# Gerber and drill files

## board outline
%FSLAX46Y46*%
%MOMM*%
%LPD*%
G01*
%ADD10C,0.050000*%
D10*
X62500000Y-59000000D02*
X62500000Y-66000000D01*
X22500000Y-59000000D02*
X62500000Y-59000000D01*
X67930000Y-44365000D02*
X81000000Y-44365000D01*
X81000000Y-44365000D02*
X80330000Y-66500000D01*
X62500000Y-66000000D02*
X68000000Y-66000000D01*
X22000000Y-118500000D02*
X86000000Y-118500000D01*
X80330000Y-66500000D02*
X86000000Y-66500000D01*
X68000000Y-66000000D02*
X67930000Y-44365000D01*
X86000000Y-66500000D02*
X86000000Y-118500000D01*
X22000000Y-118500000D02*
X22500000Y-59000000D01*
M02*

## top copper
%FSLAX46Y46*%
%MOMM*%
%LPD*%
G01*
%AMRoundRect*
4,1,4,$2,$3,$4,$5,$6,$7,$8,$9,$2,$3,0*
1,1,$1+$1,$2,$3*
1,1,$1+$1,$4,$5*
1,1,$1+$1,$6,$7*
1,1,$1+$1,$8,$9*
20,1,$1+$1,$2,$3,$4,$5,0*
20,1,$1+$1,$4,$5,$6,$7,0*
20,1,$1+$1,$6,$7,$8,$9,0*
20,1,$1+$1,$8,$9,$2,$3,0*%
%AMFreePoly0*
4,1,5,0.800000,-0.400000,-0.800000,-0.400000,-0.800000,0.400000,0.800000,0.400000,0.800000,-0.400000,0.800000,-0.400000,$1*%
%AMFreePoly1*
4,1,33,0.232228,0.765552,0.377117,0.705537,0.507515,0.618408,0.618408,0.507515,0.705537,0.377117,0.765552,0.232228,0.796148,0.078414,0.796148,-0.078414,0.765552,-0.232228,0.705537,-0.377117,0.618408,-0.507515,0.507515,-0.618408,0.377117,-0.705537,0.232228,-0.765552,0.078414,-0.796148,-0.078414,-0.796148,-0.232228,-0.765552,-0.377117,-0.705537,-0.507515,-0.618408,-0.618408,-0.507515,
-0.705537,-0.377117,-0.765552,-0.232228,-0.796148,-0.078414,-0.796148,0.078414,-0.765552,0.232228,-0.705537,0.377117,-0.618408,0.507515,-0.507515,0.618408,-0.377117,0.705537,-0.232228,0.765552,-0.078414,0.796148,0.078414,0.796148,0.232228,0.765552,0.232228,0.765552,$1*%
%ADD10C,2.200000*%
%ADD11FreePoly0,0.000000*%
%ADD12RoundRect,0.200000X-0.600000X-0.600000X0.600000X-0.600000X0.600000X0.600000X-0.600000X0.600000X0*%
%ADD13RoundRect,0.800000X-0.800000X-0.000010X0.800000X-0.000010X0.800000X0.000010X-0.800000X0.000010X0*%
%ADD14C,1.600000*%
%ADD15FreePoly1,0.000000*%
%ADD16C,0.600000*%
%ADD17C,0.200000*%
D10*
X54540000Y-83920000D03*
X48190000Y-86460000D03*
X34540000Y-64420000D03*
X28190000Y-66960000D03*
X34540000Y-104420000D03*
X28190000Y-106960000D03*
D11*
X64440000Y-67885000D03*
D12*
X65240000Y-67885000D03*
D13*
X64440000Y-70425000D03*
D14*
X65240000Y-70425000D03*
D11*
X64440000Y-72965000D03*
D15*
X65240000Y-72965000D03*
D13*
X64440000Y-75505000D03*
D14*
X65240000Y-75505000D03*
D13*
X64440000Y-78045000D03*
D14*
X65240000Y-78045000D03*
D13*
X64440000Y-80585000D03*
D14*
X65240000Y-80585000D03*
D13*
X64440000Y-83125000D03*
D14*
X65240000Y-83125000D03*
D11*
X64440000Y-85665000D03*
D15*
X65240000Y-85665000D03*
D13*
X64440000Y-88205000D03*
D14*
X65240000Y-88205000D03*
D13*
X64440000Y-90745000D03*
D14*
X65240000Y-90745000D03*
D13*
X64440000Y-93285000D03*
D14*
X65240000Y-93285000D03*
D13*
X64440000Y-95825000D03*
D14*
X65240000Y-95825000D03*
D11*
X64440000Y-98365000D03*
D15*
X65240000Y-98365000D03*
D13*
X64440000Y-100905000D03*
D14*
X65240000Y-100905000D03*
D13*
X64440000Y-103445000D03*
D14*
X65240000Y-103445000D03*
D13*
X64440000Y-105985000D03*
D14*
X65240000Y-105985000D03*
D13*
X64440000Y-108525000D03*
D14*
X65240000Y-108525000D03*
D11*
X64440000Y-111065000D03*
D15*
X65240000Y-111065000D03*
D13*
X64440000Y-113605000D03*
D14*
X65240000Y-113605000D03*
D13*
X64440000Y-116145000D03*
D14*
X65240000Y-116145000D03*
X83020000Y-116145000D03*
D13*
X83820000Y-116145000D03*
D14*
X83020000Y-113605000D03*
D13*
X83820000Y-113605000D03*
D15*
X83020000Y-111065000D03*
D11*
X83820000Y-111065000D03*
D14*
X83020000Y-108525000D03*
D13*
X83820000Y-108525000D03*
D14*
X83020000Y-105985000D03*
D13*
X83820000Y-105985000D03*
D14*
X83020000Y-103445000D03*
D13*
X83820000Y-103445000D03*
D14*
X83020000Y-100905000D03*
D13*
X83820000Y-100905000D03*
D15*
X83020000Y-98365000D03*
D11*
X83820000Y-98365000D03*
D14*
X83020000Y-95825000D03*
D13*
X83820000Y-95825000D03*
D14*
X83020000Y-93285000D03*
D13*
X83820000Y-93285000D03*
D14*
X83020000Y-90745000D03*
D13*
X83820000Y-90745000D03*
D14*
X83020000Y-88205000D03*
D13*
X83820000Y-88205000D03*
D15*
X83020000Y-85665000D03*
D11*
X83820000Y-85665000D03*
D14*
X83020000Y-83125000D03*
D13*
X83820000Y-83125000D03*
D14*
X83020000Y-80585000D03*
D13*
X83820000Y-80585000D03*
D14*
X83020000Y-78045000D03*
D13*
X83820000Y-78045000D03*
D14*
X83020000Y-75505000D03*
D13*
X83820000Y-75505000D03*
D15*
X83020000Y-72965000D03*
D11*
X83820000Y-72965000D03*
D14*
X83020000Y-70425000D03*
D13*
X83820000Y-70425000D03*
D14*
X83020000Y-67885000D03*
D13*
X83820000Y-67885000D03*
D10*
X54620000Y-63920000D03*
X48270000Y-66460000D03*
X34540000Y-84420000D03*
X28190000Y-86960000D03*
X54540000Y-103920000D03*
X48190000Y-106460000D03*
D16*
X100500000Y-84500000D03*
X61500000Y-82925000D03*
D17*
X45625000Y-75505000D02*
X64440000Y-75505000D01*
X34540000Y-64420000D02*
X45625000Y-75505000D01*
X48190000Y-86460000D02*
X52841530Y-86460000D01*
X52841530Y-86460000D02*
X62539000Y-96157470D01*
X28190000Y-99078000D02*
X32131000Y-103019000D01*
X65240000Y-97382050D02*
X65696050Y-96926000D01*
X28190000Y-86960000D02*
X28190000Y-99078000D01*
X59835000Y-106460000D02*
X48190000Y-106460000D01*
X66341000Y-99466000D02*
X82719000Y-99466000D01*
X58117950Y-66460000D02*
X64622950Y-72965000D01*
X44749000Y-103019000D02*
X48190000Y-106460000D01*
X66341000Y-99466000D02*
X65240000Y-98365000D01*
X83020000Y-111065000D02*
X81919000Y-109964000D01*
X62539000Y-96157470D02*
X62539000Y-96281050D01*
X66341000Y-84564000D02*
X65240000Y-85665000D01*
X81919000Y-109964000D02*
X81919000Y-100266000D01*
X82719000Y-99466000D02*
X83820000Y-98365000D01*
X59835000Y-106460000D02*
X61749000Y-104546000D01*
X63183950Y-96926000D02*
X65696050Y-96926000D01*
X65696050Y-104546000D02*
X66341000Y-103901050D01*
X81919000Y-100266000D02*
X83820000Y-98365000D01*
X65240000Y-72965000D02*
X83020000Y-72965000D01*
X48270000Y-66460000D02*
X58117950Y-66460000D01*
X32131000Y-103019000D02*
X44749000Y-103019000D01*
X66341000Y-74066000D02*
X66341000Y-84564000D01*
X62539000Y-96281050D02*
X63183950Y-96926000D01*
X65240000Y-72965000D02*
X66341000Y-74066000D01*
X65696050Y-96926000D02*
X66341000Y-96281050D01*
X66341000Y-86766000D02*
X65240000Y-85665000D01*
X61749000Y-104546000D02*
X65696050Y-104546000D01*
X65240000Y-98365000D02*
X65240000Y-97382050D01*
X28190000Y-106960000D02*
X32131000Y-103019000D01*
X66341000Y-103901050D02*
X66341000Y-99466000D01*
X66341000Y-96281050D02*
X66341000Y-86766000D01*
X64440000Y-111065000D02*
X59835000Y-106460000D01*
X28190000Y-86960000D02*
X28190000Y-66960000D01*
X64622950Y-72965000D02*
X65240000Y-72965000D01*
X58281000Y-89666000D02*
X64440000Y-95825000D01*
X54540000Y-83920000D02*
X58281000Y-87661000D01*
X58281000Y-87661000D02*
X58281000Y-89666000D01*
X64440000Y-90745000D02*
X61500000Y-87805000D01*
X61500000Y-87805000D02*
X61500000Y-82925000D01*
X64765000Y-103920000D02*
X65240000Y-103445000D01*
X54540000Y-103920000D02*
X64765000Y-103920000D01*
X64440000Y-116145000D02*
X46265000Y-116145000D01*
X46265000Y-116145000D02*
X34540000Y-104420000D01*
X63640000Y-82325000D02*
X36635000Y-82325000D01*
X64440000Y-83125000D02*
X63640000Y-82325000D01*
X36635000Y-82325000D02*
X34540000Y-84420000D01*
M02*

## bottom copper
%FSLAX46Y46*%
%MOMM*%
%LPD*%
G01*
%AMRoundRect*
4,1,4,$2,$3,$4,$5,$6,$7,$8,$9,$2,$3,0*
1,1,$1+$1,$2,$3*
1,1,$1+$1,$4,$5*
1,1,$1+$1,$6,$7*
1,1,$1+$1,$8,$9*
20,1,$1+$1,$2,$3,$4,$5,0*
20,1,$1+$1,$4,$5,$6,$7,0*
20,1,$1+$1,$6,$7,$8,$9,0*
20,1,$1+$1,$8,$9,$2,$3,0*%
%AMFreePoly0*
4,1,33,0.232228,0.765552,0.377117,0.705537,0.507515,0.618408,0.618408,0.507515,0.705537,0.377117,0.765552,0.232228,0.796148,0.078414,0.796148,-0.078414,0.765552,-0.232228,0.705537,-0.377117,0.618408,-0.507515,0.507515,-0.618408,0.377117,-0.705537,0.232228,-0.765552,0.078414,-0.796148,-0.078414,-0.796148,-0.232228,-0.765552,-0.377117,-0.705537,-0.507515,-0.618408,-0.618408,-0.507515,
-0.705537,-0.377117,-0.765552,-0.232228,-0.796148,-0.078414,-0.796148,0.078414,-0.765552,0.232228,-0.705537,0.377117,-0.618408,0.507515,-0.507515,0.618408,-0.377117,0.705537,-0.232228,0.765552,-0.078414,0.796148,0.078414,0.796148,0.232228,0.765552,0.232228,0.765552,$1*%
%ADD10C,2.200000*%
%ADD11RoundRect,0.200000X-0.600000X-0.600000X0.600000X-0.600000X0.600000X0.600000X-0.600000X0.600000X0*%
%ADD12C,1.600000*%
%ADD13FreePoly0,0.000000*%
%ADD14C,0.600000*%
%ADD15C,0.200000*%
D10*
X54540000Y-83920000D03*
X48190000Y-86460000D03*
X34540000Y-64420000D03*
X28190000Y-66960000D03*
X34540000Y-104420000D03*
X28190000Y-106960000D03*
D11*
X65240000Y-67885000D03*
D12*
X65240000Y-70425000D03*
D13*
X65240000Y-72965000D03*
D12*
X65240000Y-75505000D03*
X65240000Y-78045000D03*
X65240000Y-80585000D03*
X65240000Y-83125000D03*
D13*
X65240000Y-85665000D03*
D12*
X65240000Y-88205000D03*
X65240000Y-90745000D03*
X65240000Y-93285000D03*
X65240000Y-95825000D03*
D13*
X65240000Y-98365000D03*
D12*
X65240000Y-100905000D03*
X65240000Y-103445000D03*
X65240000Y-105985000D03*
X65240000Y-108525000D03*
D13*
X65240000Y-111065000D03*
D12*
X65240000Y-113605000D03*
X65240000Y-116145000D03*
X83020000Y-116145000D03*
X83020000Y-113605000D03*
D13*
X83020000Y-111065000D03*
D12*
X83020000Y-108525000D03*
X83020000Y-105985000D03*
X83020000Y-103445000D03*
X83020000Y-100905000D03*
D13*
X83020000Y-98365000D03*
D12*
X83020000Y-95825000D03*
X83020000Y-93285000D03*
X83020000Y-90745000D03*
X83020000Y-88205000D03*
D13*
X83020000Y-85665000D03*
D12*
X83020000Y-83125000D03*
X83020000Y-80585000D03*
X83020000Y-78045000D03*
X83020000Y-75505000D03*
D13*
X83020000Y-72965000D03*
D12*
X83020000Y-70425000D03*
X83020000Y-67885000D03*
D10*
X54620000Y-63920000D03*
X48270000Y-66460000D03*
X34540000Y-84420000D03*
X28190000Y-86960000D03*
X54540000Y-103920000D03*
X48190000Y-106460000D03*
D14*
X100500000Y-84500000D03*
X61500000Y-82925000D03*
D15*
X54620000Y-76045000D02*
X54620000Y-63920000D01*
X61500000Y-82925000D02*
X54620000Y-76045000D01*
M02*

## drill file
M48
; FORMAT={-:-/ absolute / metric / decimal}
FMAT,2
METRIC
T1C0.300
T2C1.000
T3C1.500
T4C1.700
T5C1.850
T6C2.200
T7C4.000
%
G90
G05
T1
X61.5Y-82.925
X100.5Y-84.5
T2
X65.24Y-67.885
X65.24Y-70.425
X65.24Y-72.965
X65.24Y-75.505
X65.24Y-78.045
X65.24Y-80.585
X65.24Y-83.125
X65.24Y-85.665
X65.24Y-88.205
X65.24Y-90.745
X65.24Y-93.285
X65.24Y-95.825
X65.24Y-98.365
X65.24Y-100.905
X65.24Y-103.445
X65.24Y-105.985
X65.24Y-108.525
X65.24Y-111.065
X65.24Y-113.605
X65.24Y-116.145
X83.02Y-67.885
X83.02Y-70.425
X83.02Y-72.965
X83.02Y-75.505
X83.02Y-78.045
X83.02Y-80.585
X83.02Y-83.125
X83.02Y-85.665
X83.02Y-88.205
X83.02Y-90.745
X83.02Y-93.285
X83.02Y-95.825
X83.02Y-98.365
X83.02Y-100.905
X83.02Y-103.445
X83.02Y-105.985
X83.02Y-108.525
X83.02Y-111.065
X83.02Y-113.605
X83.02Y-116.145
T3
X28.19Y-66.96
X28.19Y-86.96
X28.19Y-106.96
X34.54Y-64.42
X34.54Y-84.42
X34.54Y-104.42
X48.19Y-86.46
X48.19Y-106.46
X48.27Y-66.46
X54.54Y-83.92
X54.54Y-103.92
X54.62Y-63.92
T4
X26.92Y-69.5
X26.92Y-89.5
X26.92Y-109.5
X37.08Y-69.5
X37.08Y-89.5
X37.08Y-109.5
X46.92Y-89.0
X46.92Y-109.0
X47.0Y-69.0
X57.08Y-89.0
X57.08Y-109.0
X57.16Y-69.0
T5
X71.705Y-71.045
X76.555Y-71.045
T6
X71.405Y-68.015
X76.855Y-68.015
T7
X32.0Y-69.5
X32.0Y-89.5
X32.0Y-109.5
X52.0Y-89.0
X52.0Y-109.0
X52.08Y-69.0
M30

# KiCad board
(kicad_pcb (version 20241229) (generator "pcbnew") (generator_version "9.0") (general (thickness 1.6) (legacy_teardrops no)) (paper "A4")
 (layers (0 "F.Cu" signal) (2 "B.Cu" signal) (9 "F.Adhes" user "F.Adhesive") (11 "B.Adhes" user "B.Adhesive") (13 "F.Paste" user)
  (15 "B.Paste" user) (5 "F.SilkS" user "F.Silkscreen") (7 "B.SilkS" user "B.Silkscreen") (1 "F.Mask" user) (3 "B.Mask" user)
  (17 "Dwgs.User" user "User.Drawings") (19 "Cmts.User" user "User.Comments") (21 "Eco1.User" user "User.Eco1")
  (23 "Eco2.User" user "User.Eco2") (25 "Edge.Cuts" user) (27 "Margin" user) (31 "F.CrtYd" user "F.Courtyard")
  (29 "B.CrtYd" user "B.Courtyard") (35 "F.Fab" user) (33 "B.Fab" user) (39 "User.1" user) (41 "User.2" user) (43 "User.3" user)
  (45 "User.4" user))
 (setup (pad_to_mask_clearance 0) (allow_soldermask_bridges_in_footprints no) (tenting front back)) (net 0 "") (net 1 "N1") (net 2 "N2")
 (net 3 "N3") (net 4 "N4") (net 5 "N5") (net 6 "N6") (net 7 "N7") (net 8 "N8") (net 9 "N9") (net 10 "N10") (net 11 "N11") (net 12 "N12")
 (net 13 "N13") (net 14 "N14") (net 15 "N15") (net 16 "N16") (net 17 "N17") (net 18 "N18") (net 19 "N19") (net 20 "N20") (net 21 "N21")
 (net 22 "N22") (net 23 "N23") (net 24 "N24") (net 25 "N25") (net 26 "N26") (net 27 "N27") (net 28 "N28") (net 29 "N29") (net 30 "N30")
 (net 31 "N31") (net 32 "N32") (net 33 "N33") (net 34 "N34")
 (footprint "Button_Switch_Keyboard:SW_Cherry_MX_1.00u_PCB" (layer "F.Cu") (at 54.54 83.92)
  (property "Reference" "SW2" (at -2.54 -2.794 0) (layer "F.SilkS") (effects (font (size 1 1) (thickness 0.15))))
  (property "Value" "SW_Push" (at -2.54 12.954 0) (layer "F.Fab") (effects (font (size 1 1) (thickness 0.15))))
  (pad "" np_thru_hole circle (at -7.62 5.08) (size 1.7 1.7) (drill 1.7) (layers "*.Cu" "*.Mask"))
  (pad "" np_thru_hole circle (at -2.54 5.08) (size 4 4) (drill 4) (layers "*.Cu" "*.Mask"))
  (pad "" np_thru_hole circle (at 2.54 5.08) (size 1.7 1.7) (drill 1.7) (layers "*.Cu" "*.Mask"))
  (pad "1" thru_hole circle (at 0 0) (size 2.2 2.2) (drill 1.5) (layers "*.Cu" "*.Mask") (remove_unused_layers no) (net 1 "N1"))
  (pad "2" thru_hole circle (at -6.35 2.54) (size 2.2 2.2) (drill 1.5) (layers "*.Cu" "*.Mask") (remove_unused_layers no) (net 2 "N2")))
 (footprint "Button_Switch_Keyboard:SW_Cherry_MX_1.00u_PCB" (layer "F.Cu") (at 34.54 64.42)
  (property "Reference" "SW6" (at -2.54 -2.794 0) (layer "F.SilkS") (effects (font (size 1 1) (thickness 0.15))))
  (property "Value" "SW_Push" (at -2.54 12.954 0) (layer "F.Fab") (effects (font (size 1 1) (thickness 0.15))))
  (pad "" np_thru_hole circle (at -7.62 5.08) (size 1.7 1.7) (drill 1.7) (layers "*.Cu" "*.Mask"))
  (pad "" np_thru_hole circle (at -2.54 5.08) (size 4 4) (drill 4) (layers "*.Cu" "*.Mask"))
  (pad "" np_thru_hole circle (at 2.54 5.08) (size 1.7 1.7) (drill 1.7) (layers "*.Cu" "*.Mask"))
  (pad "1" thru_hole circle (at 0 0) (size 2.2 2.2) (drill 1.5) (layers "*.Cu" "*.Mask") (remove_unused_layers no) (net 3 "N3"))
  (pad "2" thru_hole circle (at -6.35 2.54) (size 2.2 2.2) (drill 1.5) (layers "*.Cu" "*.Mask") (remove_unused_layers no) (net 2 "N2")))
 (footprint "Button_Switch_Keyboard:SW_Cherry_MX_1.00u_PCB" (layer "F.Cu") (at 34.54 104.42)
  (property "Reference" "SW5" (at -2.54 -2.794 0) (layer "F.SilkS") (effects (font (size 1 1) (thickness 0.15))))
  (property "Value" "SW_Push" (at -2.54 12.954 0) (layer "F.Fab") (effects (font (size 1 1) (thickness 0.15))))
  (pad "" np_thru_hole circle (at -7.62 5.08) (size 1.7 1.7) (drill 1.7) (layers "*.Cu" "*.Mask"))
  (pad "" np_thru_hole circle (at -2.54 5.08) (size 4 4) (drill 4) (layers "*.Cu" "*.Mask"))
  (pad "" np_thru_hole circle (at 2.54 5.08) (size 1.7 1.7) (drill 1.7) (layers "*.Cu" "*.Mask"))
  (pad "1" thru_hole circle (at 0 0) (size 2.2 2.2) (drill 1.5) (layers "*.Cu" "*.Mask") (remove_unused_layers no) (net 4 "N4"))
  (pad "2" thru_hole circle (at -6.35 2.54) (size 2.2 2.2) (drill 1.5) (layers "*.Cu" "*.Mask") (remove_unused_layers no) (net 2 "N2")))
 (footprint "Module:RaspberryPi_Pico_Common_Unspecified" (layer "F.Cu") (at 74.13 92.015)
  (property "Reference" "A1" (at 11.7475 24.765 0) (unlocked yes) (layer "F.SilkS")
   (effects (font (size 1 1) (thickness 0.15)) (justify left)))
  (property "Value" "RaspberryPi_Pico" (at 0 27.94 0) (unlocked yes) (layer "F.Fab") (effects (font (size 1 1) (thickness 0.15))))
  (pad "" np_thru_hole circle (at -2.725 -24) (size 2.2 2.2) (drill 2.2) (layers "*.Mask"))
  (pad "" np_thru_hole circle (at -2.425 -20.97) (size 1.85 1.85) (drill 1.85) (layers "*.Mask"))
  (pad "" np_thru_hole circle (at 2.425 -20.97) (size 1.85 1.85) (drill 1.85) (layers "*.Mask"))
  (pad "" np_thru_hole circle (at 2.725 -24) (size 2.2 2.2) (drill 2.2) (layers "*.Mask"))
  (pad "1" smd custom (at -9.69 -24.13) (size 1.6 0.8) (layers "F.Cu" "F.Mask") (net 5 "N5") (options (clearance outline) (anchor rect))
   (primitives))
  (pad "1" thru_hole roundrect (at -8.89 -24.13) (size 1.6 1.6) (drill 1) (layers "*.Cu" "*.Mask") (remove_unused_layers no)
   (roundrect_rratio 0.125) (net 5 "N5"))
  (pad "2" smd roundrect (at -9.69 -21.59) (size 3.2 1.6) (layers "F.Cu" "F.Mask") (roundrect_rratio 0.5) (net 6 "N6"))
  (pad "2" thru_hole circle (at -8.89 -21.59) (size 1.6 1.6) (drill 1) (layers "*.Cu" "*.Mask") (remove_unused_layers no) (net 6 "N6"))
  (pad "3" smd custom (at -9.69 -19.05) (size 1.6 0.8) (layers "F.Cu" "F.Mask") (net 2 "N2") (options (clearance outline) (anchor rect))
   (primitives))
  (pad "3" thru_hole custom (at -8.89 -19.05) (size 1.6 1.6) (drill 1) (layers "*.Cu" "*.Mask") (remove_unused_layers no) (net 2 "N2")
   (options (clearance outline) (anchor circle)) (primitives))
  (pad "4" smd roundrect (at -9.69 -16.51) (size 3.2 1.6) (layers "F.Cu" "F.Mask") (roundrect_rratio 0.5) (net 3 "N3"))
  (pad "4" thru_hole circle (at -8.89 -16.51) (size 1.6 1.6) (drill 1) (layers "*.Cu" "*.Mask") (remove_unused_layers no) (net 3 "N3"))
  (pad "5" smd roundrect (at -9.69 -13.97) (size 3.2 1.6) (layers "F.Cu" "F.Mask") (roundrect_rratio 0.5) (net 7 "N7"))
  (pad "5" thru_hole circle (at -8.89 -13.97) (size 1.6 1.6) (drill 1) (layers "*.Cu" "*.Mask") (remove_unused_layers no) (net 7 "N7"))
  (pad "6" smd roundrect (at -9.69 -11.43) (size 3.2 1.6) (layers "F.Cu" "F.Mask") (roundrect_rratio 0.5) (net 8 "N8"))
  (pad "6" thru_hole circle (at -8.89 -11.43) (size 1.6 1.6) (drill 1) (layers "*.Cu" "*.Mask") (remove_unused_layers no) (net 8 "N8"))
  (pad "7" smd roundrect (at -9.69 -8.89) (size 3.2 1.6) (layers "F.Cu" "F.Mask") (roundrect_rratio 0.5) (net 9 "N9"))
  (pad "7" thru_hole circle (at -8.89 -8.89) (size 1.6 1.6) (drill 1) (layers "*.Cu" "*.Mask") (remove_unused_layers no) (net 9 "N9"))
  (pad "8" smd custom (at -9.69 -6.35) (size 1.6 0.8) (layers "F.Cu" "F.Mask") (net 2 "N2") (options (clearance outline) (anchor rect))
   (primitives))
  (pad "8" thru_hole custom (at -8.89 -6.35) (size 1.6 1.6) (drill 1) (layers "*.Cu" "*.Mask") (remove_unused_layers no) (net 2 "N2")
   (options (clearance outline) (anchor circle)) (primitives))
  (pad "9" smd roundrect (at -9.69 -3.81) (size 3.2 1.6) (layers "F.Cu" "F.Mask") (roundrect_rratio 0.5) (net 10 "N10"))
  (pad "9" thru_hole circle (at -8.89 -3.81) (size 1.6 1.6) (drill 1) (layers "*.Cu" "*.Mask") (remove_unused_layers no) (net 10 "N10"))
  (pad "10" smd roundrect (at -9.69 -1.27) (size 3.2 1.6) (layers "F.Cu" "F.Mask") (roundrect_rratio 0.5) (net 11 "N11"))
  (pad "10" thru_hole circle (at -8.89 -1.27) (size 1.6 1.6) (drill 1) (layers "*.Cu" "*.Mask") (remove_unused_layers no) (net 11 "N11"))
  (pad "11" smd roundrect (at -9.69 1.27) (size 3.2 1.6) (layers "F.Cu" "F.Mask") (roundrect_rratio 0.5) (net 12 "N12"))
  (pad "11" thru_hole circle (at -8.89 1.27) (size 1.6 1.6) (drill 1) (layers "*.Cu" "*.Mask") (remove_unused_layers no) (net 12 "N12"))
  (pad "12" smd roundrect (at -9.69 3.81) (size 3.2 1.6) (layers "F.Cu" "F.Mask") (roundrect_rratio 0.5) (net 1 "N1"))
  (pad "12" thru_hole circle (at -8.89 3.81) (size 1.6 1.6) (drill 1) (layers "*.Cu" "*.Mask") (remove_unused_layers no) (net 1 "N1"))
  (pad "13" smd custom (at -9.69 6.35) (size 1.6 0.8) (layers "F.Cu" "F.Mask") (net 2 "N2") (options (clearance outline) (anchor rect))
   (primitives))
  (pad "13" thru_hole custom (at -8.89 6.35) (size 1.6 1.6) (drill 1) (layers "*.Cu" "*.Mask") (remove_unused_layers no) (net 2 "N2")
   (options (clearance outline) (anchor circle)) (primitives))
  (pad "14" smd roundrect (at -9.69 8.89) (size 3.2 1.6) (layers "F.Cu" "F.Mask") (roundrect_rratio 0.5) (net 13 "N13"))
  (pad "14" thru_hole circle (at -8.89 8.89) (size 1.6 1.6) (drill 1) (layers "*.Cu" "*.Mask") (remove_unused_layers no) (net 13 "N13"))
  (pad "15" smd roundrect (at -9.69 11.43) (size 3.2 1.6) (layers "F.Cu" "F.Mask") (roundrect_rratio 0.5) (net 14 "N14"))
  (pad "15" thru_hole circle (at -8.89 11.43) (size 1.6 1.6) (drill 1) (layers "*.Cu" "*.Mask") (remove_unused_layers no) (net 14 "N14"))
  (pad "16" smd roundrect (at -9.69 13.97) (size 3.2 1.6) (layers "F.Cu" "F.Mask") (roundrect_rratio 0.5) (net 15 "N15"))
  (pad "16" thru_hole circle (at -8.89 13.97) (size 1.6 1.6) (drill 1) (layers "*.Cu" "*.Mask") (remove_unused_layers no) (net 15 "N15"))
  (pad "17" smd roundrect (at -9.69 16.51) (size 3.2 1.6) (layers "F.Cu" "F.Mask") (roundrect_rratio 0.5) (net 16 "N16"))
  (pad "17" thru_hole circle (at -8.89 16.51) (size 1.6 1.6) (drill 1) (layers "*.Cu" "*.Mask") (remove_unused_layers no) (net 16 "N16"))
  (pad "18" smd custom (at -9.69 19.05) (size 1.6 0.8) (layers "F.Cu" "F.Mask") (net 2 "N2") (options (clearance outline) (anchor rect))
   (primitives))
  (pad "18" thru_hole custom (at -8.89 19.05) (size 1.6 1.6) (drill 1) (layers "*.Cu" "*.Mask") (remove_unused_layers no) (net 2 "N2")
   (options (clearance outline) (anchor circle)) (primitives))
  (pad "19" smd roundrect (at -9.69 21.59) (size 3.2 1.6) (layers "F.Cu" "F.Mask") (roundrect_rratio 0.5) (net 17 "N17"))
  (pad "19" thru_hole circle (at -8.89 21.59) (size 1.6 1.6) (drill 1) (layers "*.Cu" "*.Mask") (remove_unused_layers no) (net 17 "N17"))
  (pad "20" smd roundrect (at -9.69 24.13) (size 3.2 1.6) (layers "F.Cu" "F.Mask") (roundrect_rratio 0.5) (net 4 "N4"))
  (pad "20" thru_hole circle (at -8.89 24.13) (size 1.6 1.6) (drill 1) (layers "*.Cu" "*.Mask") (remove_unused_layers no) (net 4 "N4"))
  (pad "21" thru_hole circle (at 8.89 24.13) (size 1.6 1.6) (drill 1) (layers "*.Cu" "*.Mask") (remove_unused_layers no) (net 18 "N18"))
  (pad "21" smd roundrect (at 9.69 24.13) (size 3.2 1.6) (layers "F.Cu" "F.Mask") (roundrect_rratio 0.5) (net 18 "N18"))
  (pad "22" thru_hole circle (at 8.89 21.59) (size 1.6 1.6) (drill 1) (layers "*.Cu" "*.Mask") (remove_unused_layers no) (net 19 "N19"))
  (pad "22" smd roundrect (at 9.69 21.59) (size 3.2 1.6) (layers "F.Cu" "F.Mask") (roundrect_rratio 0.5) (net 19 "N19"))
  (pad "23" thru_hole custom (at 8.89 19.05) (size 1.6 1.6) (drill 1) (layers "*.Cu" "*.Mask") (remove_unused_layers no) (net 2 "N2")
   (options (clearance outline) (anchor circle)) (primitives))
  (pad "23" smd custom (at 9.69 19.05) (size 1.6 0.8) (layers "F.Cu" "F.Mask") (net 2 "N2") (options (clearance outline) (anchor rect))
   (primitives))
  (pad "24" thru_hole circle (at 8.89 16.51) (size 1.6 1.6) (drill 1) (layers "*.Cu" "*.Mask") (remove_unused_layers no) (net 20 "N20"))
  (pad "24" smd roundrect (at 9.69 16.51) (size 3.2 1.6) (layers "F.Cu" "F.Mask") (roundrect_rratio 0.5) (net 20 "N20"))
  (pad "25" thru_hole circle (at 8.89 13.97) (size 1.6 1.6) (drill 1) (layers "*.Cu" "*.Mask") (remove_unused_layers no) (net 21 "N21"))
  (pad "25" smd roundrect (at 9.69 13.97) (size 3.2 1.6) (layers "F.Cu" "F.Mask") (roundrect_rratio 0.5) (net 21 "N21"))
  (pad "26" thru_hole circle (at 8.89 11.43) (size 1.6 1.6) (drill 1) (layers "*.Cu" "*.Mask") (remove_unused_layers no) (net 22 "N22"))
  (pad "26" smd roundrect (at 9.69 11.43) (size 3.2 1.6) (layers "F.Cu" "F.Mask") (roundrect_rratio 0.5) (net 22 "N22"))
  (pad "27" thru_hole circle (at 8.89 8.89) (size 1.6 1.6) (drill 1) (layers "*.Cu" "*.Mask") (remove_unused_layers no) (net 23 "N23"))
  (pad "27" smd roundrect (at 9.69 8.89) (size 3.2 1.6) (layers "F.Cu" "F.Mask") (roundrect_rratio 0.5) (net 23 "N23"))
  (pad "28" thru_hole custom (at 8.89 6.35) (size 1.6 1.6) (drill 1) (layers "*.Cu" "*.Mask") (remove_unused_layers no) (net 2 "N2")
   (options (clearance outline) (anchor circle)) (primitives))
  (pad "28" smd custom (at 9.69 6.35) (size 1.6 0.8) (layers "F.Cu" "F.Mask") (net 2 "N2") (options (clearance outline) (anchor rect))
   (primitives))
  (pad "29" thru_hole circle (at 8.89 3.81) (size 1.6 1.6) (drill 1) (layers "*.Cu" "*.Mask") (remove_unused_layers no) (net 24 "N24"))
  (pad "29" smd roundrect (at 9.69 3.81) (size 3.2 1.6) (layers "F.Cu" "F.Mask") (roundrect_rratio 0.5) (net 24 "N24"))
  (pad "30" thru_hole circle (at 8.89 1.27) (size 1.6 1.6) (drill 1) (layers "*.Cu" "*.Mask") (remove_unused_layers no) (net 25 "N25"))
  (pad "30" smd roundrect (at 9.69 1.27) (size 3.2 1.6) (layers "F.Cu" "F.Mask") (roundrect_rratio 0.5) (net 25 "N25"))
  (pad "31" thru_hole circle (at 8.89 -1.27) (size 1.6 1.6) (drill 1) (layers "*.Cu" "*.Mask") (remove_unused_layers no) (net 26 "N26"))
  (pad "31" smd roundrect (at 9.69 -1.27) (size 3.2 1.6) (layers "F.Cu" "F.Mask") (roundrect_rratio 0.5) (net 26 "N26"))
  (pad "32" thru_hole circle (at 8.89 -3.81) (size 1.6 1.6) (drill 1) (layers "*.Cu" "*.Mask") (remove_unused_layers no) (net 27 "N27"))
  (pad "32" smd roundrect (at 9.69 -3.81) (size 3.2 1.6) (layers "F.Cu" "F.Mask") (roundrect_rratio 0.5) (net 27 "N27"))
  (pad "33" thru_hole custom (at 8.89 -6.35) (size 1.6 1.6) (drill 1) (layers "*.Cu" "*.Mask") (remove_unused_layers no) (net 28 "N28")
   (options (clearance outline) (anchor circle)) (primitives))
  (pad "33" smd custom (at 9.69 -6.35) (size 1.6 0.8) (layers "F.Cu" "F.Mask") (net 28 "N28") (options (clearance outline) (anchor rect))
   (primitives))
  (pad "34" thru_hole circle (at 8.89 -8.89) (size 1.6 1.6) (drill 1) (layers "*.Cu" "*.Mask") (remove_unused_layers no) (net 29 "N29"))
  (pad "34" smd roundrect (at 9.69 -8.89) (size 3.2 1.6) (layers "F.Cu" "F.Mask") (roundrect_rratio 0.5) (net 29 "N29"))
  (pad "35" thru_hole circle (at 8.89 -11.43) (size 1.6 1.6) (drill 1) (layers "*.Cu" "*.Mask") (remove_unused_layers no) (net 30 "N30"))
  (pad "35" smd roundrect (at 9.69 -11.43) (size 3.2 1.6) (layers "F.Cu" "F.Mask") (roundrect_rratio 0.5) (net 30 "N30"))
  (pad "36" thru_hole circle (at 8.89 -13.97) (size 1.6 1.6) (drill 1) (layers "*.Cu" "*.Mask") (remove_unused_layers no) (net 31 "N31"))
  (pad "36" smd roundrect (at 9.69 -13.97) (size 3.2 1.6) (layers "F.Cu" "F.Mask") (roundrect_rratio 0.5) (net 31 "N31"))
  (pad "37" thru_hole circle (at 8.89 -16.51) (size 1.6 1.6) (drill 1) (layers "*.Cu" "*.Mask") (remove_unused_layers no) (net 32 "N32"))
  (pad "37" smd roundrect (at 9.69 -16.51) (size 3.2 1.6) (layers "F.Cu" "F.Mask") (roundrect_rratio 0.5) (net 32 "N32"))
  (pad "38" thru_hole custom (at 8.89 -19.05) (size 1.6 1.6) (drill 1) (layers "*.Cu" "*.Mask") (remove_unused_layers no) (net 2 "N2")
   (options (clearance outline) (anchor circle)) (primitives))
  (pad "38" smd custom (at 9.69 -19.05) (size 1.6 0.8) (layers "F.Cu" "F.Mask") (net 2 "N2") (options (clearance outline) (anchor rect))
   (primitives))
  (pad "39" thru_hole circle (at 8.89 -21.59) (size 1.6 1.6) (drill 1) (layers "*.Cu" "*.Mask") (remove_unused_layers no) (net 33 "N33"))
  (pad "39" smd roundrect (at 9.69 -21.59) (size 3.2 1.6) (layers "F.Cu" "F.Mask") (roundrect_rratio 0.5) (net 33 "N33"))
  (pad "40" thru_hole circle (at 8.89 -24.13) (size 1.6 1.6) (drill 1) (layers "*.Cu" "*.Mask") (remove_unused_layers no) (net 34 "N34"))
  (pad "40" smd roundrect (at 9.69 -24.13) (size 3.2 1.6) (layers "F.Cu" "F.Mask") (roundrect_rratio 0.5) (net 34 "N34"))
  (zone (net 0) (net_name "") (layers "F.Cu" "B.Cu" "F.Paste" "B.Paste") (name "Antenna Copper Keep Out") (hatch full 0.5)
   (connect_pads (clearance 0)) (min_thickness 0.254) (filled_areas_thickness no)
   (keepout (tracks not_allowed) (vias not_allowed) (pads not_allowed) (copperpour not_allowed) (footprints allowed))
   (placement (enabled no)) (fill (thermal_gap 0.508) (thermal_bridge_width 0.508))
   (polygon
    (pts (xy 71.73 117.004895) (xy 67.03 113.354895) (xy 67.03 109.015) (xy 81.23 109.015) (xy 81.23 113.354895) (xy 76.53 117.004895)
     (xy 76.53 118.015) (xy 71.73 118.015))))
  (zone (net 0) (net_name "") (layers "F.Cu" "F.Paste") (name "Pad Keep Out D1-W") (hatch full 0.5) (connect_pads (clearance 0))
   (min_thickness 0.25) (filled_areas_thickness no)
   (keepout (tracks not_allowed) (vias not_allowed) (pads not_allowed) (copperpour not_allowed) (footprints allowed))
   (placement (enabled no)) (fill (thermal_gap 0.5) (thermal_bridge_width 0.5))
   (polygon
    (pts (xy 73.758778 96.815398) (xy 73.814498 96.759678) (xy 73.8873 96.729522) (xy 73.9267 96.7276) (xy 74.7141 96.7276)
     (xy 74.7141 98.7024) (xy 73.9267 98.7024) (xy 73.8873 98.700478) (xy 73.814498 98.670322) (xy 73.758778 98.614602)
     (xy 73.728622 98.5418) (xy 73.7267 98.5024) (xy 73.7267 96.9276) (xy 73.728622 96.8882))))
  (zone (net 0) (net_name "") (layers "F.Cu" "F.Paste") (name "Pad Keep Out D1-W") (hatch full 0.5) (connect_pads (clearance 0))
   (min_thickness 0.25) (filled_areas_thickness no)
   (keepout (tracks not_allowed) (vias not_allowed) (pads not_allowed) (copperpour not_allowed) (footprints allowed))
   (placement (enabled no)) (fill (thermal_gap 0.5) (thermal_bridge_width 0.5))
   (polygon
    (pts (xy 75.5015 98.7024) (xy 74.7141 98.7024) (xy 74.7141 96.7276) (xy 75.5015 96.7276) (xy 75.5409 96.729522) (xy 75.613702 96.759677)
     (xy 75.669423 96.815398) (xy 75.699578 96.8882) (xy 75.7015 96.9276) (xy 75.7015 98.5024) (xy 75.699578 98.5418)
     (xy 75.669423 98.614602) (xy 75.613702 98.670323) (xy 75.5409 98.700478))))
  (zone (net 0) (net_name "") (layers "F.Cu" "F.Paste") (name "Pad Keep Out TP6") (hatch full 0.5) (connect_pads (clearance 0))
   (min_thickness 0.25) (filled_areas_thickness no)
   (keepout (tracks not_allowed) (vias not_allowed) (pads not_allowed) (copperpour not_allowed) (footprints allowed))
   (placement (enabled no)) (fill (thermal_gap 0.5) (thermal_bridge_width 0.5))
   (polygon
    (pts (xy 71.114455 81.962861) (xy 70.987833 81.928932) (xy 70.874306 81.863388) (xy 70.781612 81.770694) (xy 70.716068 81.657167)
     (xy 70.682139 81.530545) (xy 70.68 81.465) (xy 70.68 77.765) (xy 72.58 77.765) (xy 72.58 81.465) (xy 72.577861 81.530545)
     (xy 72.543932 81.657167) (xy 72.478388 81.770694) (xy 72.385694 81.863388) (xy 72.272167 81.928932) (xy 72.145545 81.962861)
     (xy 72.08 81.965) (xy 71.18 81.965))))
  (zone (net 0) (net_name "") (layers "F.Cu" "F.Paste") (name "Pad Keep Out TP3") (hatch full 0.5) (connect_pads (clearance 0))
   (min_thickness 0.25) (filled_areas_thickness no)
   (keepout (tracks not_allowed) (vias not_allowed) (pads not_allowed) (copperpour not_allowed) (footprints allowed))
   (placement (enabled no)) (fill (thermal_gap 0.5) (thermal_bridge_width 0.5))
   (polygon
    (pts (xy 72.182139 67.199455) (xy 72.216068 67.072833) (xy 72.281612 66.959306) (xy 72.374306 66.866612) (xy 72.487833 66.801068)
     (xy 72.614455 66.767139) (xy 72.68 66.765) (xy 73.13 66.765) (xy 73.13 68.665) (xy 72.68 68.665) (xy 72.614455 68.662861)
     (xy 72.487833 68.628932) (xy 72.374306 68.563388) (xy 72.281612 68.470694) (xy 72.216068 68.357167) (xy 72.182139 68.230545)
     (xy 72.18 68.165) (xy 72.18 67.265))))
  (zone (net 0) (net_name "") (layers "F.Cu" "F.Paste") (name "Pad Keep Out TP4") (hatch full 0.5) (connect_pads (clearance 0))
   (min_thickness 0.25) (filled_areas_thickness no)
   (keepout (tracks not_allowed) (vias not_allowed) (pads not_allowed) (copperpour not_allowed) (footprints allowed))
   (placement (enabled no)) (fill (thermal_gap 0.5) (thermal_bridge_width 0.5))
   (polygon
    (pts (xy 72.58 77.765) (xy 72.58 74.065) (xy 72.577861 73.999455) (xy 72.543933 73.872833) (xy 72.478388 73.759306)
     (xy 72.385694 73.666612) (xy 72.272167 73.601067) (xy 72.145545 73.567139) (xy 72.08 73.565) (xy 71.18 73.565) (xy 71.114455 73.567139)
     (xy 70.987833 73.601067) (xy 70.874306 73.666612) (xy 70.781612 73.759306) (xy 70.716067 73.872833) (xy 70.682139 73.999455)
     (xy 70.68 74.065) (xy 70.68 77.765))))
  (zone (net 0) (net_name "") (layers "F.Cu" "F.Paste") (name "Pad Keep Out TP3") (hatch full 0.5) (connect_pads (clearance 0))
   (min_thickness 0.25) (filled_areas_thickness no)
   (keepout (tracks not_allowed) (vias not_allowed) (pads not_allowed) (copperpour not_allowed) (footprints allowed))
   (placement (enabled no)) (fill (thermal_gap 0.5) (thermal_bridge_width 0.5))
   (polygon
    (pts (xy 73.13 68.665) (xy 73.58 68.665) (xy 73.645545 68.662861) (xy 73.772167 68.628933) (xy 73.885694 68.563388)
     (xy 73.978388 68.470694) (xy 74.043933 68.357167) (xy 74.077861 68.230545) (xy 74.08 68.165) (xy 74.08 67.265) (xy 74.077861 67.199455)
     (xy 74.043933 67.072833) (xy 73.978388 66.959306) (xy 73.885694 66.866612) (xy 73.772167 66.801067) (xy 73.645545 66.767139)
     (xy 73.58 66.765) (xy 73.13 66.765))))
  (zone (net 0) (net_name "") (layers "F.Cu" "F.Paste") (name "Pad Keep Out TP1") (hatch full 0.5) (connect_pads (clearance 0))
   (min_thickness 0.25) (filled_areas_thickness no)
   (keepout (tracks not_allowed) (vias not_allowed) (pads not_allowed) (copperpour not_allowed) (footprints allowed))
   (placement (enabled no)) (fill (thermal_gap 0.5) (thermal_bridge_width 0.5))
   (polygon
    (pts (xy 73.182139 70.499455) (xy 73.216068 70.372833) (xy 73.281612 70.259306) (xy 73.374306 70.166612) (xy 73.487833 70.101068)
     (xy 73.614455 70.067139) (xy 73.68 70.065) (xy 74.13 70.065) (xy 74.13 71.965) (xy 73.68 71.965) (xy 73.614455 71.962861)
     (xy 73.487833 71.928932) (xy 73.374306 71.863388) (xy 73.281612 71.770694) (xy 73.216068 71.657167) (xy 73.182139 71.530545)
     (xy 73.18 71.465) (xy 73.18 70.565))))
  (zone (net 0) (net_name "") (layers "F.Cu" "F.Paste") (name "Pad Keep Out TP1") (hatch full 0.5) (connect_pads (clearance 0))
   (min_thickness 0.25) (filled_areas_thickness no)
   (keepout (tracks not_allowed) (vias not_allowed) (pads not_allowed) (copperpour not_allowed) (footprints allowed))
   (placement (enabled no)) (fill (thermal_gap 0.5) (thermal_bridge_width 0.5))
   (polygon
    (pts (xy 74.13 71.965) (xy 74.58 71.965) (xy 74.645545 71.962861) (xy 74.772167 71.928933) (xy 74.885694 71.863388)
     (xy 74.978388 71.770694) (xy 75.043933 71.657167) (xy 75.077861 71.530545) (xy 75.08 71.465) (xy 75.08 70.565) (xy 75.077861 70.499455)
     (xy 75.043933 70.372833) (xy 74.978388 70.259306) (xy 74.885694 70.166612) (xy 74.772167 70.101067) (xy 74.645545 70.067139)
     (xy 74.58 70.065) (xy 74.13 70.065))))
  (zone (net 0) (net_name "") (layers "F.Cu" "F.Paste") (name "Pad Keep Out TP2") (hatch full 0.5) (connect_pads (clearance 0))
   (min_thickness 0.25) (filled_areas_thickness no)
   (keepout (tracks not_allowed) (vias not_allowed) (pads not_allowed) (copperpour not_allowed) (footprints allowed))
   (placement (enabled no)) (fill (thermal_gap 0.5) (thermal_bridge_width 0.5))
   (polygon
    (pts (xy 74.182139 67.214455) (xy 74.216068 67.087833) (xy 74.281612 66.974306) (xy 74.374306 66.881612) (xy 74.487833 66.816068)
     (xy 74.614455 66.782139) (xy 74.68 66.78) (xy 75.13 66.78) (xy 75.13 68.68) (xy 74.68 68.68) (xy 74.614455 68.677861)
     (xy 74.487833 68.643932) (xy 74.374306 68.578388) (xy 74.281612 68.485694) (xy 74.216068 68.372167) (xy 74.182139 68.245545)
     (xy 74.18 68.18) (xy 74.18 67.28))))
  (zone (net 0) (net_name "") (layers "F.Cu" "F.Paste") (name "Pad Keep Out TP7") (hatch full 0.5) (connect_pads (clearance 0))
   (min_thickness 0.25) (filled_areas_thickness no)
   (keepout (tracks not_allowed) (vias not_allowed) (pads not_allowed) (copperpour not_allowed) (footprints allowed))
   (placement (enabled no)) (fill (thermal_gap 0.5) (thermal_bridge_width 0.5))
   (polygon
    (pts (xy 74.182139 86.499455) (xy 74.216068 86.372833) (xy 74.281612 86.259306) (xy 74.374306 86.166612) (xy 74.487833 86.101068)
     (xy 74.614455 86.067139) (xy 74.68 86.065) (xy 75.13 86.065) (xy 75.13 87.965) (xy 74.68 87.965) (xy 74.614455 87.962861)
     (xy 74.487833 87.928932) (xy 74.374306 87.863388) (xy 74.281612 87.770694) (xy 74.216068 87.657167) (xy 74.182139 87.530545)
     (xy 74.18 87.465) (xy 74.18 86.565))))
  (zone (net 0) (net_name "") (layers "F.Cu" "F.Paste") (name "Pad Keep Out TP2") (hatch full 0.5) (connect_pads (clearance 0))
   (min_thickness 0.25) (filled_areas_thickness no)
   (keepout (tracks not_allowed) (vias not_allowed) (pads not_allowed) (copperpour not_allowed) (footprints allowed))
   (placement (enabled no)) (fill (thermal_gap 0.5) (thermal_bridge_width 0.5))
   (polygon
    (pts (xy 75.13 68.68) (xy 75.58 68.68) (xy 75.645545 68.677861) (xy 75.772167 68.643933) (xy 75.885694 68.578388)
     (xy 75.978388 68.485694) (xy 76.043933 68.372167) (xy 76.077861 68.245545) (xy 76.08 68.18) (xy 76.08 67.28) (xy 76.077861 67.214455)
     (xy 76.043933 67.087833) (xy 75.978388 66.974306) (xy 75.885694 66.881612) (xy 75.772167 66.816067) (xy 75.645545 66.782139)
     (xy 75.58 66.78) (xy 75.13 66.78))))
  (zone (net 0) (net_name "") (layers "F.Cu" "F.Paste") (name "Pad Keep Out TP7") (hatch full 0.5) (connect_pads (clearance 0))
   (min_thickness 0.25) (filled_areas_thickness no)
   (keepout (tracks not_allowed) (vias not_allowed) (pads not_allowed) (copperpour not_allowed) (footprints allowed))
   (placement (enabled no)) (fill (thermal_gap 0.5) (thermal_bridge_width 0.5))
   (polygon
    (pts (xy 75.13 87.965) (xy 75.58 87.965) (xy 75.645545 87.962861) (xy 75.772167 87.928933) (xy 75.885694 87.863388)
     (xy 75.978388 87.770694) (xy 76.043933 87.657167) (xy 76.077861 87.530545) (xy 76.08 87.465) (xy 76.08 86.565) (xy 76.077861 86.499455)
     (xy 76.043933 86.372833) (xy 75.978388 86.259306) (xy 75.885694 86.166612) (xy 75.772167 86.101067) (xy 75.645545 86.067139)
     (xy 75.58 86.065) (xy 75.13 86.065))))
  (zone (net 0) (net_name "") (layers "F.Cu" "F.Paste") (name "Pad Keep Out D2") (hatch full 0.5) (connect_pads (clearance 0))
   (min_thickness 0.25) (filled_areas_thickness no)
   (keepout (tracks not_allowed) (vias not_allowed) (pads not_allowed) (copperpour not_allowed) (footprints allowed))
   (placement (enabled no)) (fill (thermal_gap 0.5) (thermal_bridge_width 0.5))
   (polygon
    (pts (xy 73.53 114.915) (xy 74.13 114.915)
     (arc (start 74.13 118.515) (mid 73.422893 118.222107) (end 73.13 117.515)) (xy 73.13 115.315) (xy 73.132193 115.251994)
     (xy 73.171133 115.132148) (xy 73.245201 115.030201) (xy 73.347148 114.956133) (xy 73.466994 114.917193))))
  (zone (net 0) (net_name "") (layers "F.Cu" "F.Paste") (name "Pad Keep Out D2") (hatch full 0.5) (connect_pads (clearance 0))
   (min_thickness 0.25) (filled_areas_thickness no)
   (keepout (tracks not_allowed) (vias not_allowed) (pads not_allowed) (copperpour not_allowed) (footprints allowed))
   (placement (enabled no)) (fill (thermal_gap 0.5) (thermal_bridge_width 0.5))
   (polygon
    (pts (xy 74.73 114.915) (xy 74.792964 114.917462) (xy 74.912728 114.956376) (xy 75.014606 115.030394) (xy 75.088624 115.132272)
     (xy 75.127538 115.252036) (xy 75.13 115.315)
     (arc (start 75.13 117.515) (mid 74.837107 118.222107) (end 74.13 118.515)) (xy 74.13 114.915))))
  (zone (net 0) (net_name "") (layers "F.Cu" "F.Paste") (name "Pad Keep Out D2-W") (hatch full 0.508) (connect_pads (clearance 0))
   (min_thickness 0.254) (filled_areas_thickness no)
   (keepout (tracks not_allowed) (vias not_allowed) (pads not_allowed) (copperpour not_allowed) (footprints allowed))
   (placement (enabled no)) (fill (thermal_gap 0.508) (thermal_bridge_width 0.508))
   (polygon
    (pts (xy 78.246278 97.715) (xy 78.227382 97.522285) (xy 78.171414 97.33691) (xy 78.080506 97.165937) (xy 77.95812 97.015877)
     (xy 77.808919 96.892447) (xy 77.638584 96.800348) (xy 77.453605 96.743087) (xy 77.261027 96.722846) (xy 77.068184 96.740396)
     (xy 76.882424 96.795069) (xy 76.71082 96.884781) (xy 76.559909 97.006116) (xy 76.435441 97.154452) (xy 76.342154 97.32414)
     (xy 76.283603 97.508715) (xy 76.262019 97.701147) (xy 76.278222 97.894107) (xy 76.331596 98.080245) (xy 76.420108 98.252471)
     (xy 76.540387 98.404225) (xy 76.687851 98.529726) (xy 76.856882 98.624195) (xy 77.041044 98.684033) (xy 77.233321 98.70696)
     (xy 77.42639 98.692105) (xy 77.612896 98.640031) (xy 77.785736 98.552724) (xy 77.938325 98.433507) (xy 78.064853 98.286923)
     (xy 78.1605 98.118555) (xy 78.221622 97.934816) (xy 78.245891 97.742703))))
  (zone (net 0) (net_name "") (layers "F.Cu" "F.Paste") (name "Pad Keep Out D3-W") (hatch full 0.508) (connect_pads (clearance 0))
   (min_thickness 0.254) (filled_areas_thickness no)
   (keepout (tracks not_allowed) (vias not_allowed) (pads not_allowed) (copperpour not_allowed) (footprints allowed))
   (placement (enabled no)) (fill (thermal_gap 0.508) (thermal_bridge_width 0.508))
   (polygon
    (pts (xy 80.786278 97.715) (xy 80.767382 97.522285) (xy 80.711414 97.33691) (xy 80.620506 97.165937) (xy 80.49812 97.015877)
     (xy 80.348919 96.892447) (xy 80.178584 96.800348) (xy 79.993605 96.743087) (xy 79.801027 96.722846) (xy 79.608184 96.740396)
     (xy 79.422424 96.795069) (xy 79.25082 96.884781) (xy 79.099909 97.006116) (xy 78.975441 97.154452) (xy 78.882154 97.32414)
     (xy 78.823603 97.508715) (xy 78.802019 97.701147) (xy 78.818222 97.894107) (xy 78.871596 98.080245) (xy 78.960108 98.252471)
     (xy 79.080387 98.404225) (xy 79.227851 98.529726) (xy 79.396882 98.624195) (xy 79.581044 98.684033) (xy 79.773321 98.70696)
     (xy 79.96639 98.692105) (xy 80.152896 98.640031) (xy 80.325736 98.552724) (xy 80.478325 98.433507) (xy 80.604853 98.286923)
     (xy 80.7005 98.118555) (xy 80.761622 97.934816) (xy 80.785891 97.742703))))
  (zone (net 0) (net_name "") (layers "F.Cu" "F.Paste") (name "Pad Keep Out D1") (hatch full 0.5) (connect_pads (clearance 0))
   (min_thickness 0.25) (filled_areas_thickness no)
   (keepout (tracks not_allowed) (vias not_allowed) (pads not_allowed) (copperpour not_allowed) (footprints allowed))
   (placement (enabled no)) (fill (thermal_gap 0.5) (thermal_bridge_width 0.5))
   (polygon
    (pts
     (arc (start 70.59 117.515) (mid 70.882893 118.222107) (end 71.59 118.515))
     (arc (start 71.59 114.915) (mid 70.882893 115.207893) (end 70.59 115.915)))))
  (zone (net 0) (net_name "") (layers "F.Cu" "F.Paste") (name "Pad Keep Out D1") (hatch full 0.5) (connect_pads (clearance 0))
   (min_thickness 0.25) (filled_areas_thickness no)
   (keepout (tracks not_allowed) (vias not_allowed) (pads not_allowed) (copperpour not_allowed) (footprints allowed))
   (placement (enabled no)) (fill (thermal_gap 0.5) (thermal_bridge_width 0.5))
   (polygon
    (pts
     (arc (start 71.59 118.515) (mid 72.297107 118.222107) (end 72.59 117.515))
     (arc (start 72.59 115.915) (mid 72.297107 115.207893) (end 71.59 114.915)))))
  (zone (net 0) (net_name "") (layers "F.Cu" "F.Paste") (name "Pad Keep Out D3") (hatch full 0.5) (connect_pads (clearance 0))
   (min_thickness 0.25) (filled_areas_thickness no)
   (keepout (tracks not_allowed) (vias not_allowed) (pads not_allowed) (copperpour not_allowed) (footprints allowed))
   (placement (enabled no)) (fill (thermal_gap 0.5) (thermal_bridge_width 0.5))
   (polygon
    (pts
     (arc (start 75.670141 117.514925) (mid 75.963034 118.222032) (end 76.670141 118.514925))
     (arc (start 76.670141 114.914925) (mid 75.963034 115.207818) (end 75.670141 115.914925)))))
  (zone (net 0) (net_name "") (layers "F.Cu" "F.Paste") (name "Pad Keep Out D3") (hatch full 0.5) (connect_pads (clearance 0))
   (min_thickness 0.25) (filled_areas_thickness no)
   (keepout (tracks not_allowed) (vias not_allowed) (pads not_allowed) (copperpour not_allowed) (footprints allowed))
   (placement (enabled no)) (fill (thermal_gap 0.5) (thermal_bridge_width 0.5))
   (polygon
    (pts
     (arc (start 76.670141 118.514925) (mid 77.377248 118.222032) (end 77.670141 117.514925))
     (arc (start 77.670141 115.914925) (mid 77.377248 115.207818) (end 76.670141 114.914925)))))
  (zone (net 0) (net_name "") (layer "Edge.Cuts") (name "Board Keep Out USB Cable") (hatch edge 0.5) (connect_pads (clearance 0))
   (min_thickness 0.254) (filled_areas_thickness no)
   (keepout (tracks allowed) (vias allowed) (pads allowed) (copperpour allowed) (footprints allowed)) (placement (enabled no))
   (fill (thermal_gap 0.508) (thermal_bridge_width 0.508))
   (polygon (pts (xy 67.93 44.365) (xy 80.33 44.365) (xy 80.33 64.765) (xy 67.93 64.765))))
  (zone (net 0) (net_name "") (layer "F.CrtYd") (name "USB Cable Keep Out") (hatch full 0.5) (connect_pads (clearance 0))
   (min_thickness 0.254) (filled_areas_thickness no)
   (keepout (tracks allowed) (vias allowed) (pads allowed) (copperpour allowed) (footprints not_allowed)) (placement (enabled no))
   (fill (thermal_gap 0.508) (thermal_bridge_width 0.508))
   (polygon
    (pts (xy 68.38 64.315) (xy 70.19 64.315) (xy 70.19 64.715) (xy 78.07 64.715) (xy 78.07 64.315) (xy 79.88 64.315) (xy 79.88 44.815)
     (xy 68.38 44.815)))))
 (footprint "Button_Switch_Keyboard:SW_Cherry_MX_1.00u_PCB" (layer "F.Cu") (at 54.62 63.92)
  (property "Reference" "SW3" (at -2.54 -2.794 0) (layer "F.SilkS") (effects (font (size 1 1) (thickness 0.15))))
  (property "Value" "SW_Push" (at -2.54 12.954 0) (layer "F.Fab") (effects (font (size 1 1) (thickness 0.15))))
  (pad "" np_thru_hole circle (at -7.62 5.08) (size 1.7 1.7) (drill 1.7) (layers "*.Cu" "*.Mask"))
  (pad "" np_thru_hole circle (at -2.54 5.08) (size 4 4) (drill 4) (layers "*.Cu" "*.Mask"))
  (pad "" np_thru_hole circle (at 2.54 5.08) (size 1.7 1.7) (drill 1.7) (layers "*.Cu" "*.Mask"))
  (pad "1" thru_hole circle (at 0 0) (size 2.2 2.2) (drill 1.5) (layers "*.Cu" "*.Mask") (remove_unused_layers no) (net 11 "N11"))
  (pad "2" thru_hole circle (at -6.35 2.54) (size 2.2 2.2) (drill 1.5) (layers "*.Cu" "*.Mask") (remove_unused_layers no) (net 2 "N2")))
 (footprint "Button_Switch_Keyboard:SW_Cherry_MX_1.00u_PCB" (layer "F.Cu") (at 34.54 84.42)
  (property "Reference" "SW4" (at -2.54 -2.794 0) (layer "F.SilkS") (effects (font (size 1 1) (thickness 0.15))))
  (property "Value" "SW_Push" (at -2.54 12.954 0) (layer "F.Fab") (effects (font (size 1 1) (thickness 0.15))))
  (pad "" np_thru_hole circle (at -7.62 5.08) (size 1.7 1.7) (drill 1.7) (layers "*.Cu" "*.Mask"))
  (pad "" np_thru_hole circle (at -2.54 5.08) (size 4 4) (drill 4) (layers "*.Cu" "*.Mask"))
  (pad "" np_thru_hole circle (at 2.54 5.08) (size 1.7 1.7) (drill 1.7) (layers "*.Cu" "*.Mask"))
  (pad "1" thru_hole circle (at 0 0) (size 2.2 2.2) (drill 1.5) (layers "*.Cu" "*.Mask") (remove_unused_layers no) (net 9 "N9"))
  (pad "2" thru_hole circle (at -6.35 2.54) (size 2.2 2.2) (drill 1.5) (layers "*.Cu" "*.Mask") (remove_unused_layers no) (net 2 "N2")))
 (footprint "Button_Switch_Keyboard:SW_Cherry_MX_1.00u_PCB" (layer "F.Cu") (at 54.54 103.92)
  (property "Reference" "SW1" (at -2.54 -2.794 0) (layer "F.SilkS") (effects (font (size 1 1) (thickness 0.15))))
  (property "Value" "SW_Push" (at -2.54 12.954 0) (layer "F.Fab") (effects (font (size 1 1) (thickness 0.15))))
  (pad "" np_thru_hole circle (at -7.62 5.08) (size 1.7 1.7) (drill 1.7) (layers "*.Cu" "*.Mask"))
  (pad "" np_thru_hole circle (at -2.54 5.08) (size 4 4) (drill 4) (layers "*.Cu" "*.Mask"))
  (pad "" np_thru_hole circle (at 2.54 5.08) (size 1.7 1.7) (drill 1.7) (layers "*.Cu" "*.Mask"))
  (pad "1" thru_hole circle (at 0 0) (size 2.2 2.2) (drill 1.5) (layers "*.Cu" "*.Mask") (remove_unused_layers no) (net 14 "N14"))
  (pad "2" thru_hole circle (at -6.35 2.54) (size 2.2 2.2) (drill 1.5) (layers "*.Cu" "*.Mask") (remove_unused_layers no) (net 2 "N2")))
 (gr_line (start 62.5 59) (end 62.5 66) (stroke (width 0.05) (type default)) (layer "Edge.Cuts"))
 (gr_line (start 22.5 59) (end 62.5 59) (stroke (width 0.05) (type default)) (layer "Edge.Cuts"))
 (gr_line (start 67.93 44.365) (end 81 44.365) (stroke (width 0.05) (type default)) (layer "Edge.Cuts"))
 (gr_line (start 81 44.365) (end 80.33 66.5) (stroke (width 0.05) (type default)) (layer "Edge.Cuts"))
 (gr_line (start 62.5 66) (end 68 66) (stroke (width 0.05) (type default)) (layer "Edge.Cuts"))
 (gr_line (start 22 118.5) (end 86 118.5) (stroke (width 0.05) (type default)) (layer "Edge.Cuts"))
 (gr_line (start 80.33 66.5) (end 86 66.5) (stroke (width 0.05) (type default)) (layer "Edge.Cuts"))
 (gr_line (start 68 66) (end 67.93 44.365) (stroke (width 0.05) (type default)) (layer "Edge.Cuts"))
 (gr_line (start 86 66.5) (end 86 118.5) (stroke (width 0.05) (type default)) (layer "Edge.Cuts"))
 (gr_line (start 22 118.5) (end 22.5 59) (stroke (width 0.05) (type default)) (layer "Edge.Cuts"))
 (via (at 100.5 84.5) (size 0.6) (drill 0.3) (layers "F.Cu" "B.Cu") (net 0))
 (segment (start 45.625 75.505) (end 64.44 75.505) (width 0.2) (layer "F.Cu") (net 3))
 (segment (start 34.54 64.42) (end 45.625 75.505) (width 0.2) (layer "F.Cu") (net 3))
 (segment (start 48.19 86.46) (end 52.84153 86.46) (width 0.2) (layer "F.Cu") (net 2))
 (segment (start 52.84153 86.46) (end 62.539 96.15747) (width 0.2) (layer "F.Cu") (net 2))
 (segment (start 28.19 99.078) (end 32.131 103.019) (width 0.2) (layer "F.Cu") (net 2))
 (segment (start 65.24 97.38205) (end 65.69605 96.926) (width 0.2) (layer "F.Cu") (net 2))
 (segment (start 28.19 86.96) (end 28.19 99.078) (width 0.2) (layer "F.Cu") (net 2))
 (segment (start 59.835 106.46) (end 48.19 106.46) (width 0.2) (layer "F.Cu") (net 2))
 (segment (start 66.341 99.466) (end 82.719 99.466) (width 0.2) (layer "F.Cu") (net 2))
 (segment (start 58.11795 66.46) (end 64.62295 72.965) (width 0.2) (layer "F.Cu") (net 2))
 (segment (start 44.749 103.019) (end 48.19 106.46) (width 0.2) (layer "F.Cu") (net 2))
 (segment (start 66.341 99.466) (end 65.24 98.365) (width 0.2) (layer "F.Cu") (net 2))
 (segment (start 83.02 111.065) (end 81.919 109.964) (width 0.2) (layer "F.Cu") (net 2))
 (segment (start 62.539 96.15747) (end 62.539 96.28105) (width 0.2) (layer "F.Cu") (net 2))
 (segment (start 66.341 84.564) (end 65.24 85.665) (width 0.2) (layer "F.Cu") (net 2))
 (segment (start 81.919 109.964) (end 81.919 100.266) (width 0.2) (layer "F.Cu") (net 2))
 (segment (start 82.719 99.466) (end 83.82 98.365) (width 0.2) (layer "F.Cu") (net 2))
 (segment (start 59.835 106.46) (end 61.749 104.546) (width 0.2) (layer "F.Cu") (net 2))
 (segment (start 63.18395 96.926) (end 65.69605 96.926) (width 0.2) (layer "F.Cu") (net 2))
 (segment (start 65.69605 104.546) (end 66.341 103.90105) (width 0.2) (layer "F.Cu") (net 2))
 (segment (start 81.919 100.266) (end 83.82 98.365) (width 0.2) (layer "F.Cu") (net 2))
 (segment (start 65.24 72.965) (end 83.02 72.965) (width 0.2) (layer "F.Cu") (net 2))
 (segment (start 48.27 66.46) (end 58.11795 66.46) (width 0.2) (layer "F.Cu") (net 2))
 (segment (start 32.131 103.019) (end 44.749 103.019) (width 0.2) (layer "F.Cu") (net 2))
 (segment (start 66.341 74.066) (end 66.341 84.564) (width 0.2) (layer "F.Cu") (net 2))
 (segment (start 62.539 96.28105) (end 63.18395 96.926) (width 0.2) (layer "F.Cu") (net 2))
 (segment (start 65.24 72.965) (end 66.341 74.066) (width 0.2) (layer "F.Cu") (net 2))
 (segment (start 65.69605 96.926) (end 66.341 96.28105) (width 0.2) (layer "F.Cu") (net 2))
 (segment (start 66.341 86.766) (end 65.24 85.665) (width 0.2) (layer "F.Cu") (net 2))
 (segment (start 61.749 104.546) (end 65.69605 104.546) (width 0.2) (layer "F.Cu") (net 2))
 (segment (start 65.24 98.365) (end 65.24 97.38205) (width 0.2) (layer "F.Cu") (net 2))
 (segment (start 28.19 106.96) (end 32.131 103.019) (width 0.2) (layer "F.Cu") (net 2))
 (segment (start 66.341 103.90105) (end 66.341 99.466) (width 0.2) (layer "F.Cu") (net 2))
 (segment (start 66.341 96.28105) (end 66.341 86.766) (width 0.2) (layer "F.Cu") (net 2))
 (segment (start 64.44 111.065) (end 59.835 106.46) (width 0.2) (layer "F.Cu") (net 2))
 (segment (start 28.19 86.96) (end 28.19 66.96) (width 0.2) (layer "F.Cu") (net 2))
 (segment (start 64.62295 72.965) (end 65.24 72.965) (width 0.2) (layer "F.Cu") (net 2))
 (segment (start 58.281 89.666) (end 64.44 95.825) (width 0.2) (layer "F.Cu") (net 1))
 (segment (start 54.54 83.92) (end 58.281 87.661) (width 0.2) (layer "F.Cu") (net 1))
 (segment (start 58.281 87.661) (end 58.281 89.666) (width 0.2) (layer "F.Cu") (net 1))
 (segment (start 64.44 90.745) (end 61.5 87.805) (width 0.2) (layer "F.Cu") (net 11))
 (segment (start 61.5 87.805) (end 61.5 82.925) (width 0.2) (layer "F.Cu") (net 11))
 (via (at 61.5 82.925) (size 0.6) (drill 0.3) (layers "F.Cu" "B.Cu") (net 11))
 (segment (start 54.62 76.045) (end 54.62 63.92) (width 0.2) (layer "B.Cu") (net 11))
 (segment (start 61.5 82.925) (end 54.62 76.045) (width 0.2) (layer "B.Cu") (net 11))
 (segment (start 64.765 103.92) (end 65.24 103.445) (width 0.2) (layer "F.Cu") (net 14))
 (segment (start 54.54 103.92) (end 64.765 103.92) (width 0.2) (layer "F.Cu") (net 14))
 (segment (start 64.44 116.145) (end 46.265 116.145) (width 0.2) (layer "F.Cu") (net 4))
 (segment (start 46.265 116.145) (end 34.54 104.42) (width 0.2) (layer "F.Cu") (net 4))
 (segment (start 63.64 82.325) (end 36.635 82.325) (width 0.2) (layer "F.Cu") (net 9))
 (segment (start 64.44 83.125) (end 63.64 82.325) (width 0.2) (layer "F.Cu") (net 9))
 (segment (start 36.635 82.325) (end 34.54 84.42) (width 0.2) (layer "F.Cu") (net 9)))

